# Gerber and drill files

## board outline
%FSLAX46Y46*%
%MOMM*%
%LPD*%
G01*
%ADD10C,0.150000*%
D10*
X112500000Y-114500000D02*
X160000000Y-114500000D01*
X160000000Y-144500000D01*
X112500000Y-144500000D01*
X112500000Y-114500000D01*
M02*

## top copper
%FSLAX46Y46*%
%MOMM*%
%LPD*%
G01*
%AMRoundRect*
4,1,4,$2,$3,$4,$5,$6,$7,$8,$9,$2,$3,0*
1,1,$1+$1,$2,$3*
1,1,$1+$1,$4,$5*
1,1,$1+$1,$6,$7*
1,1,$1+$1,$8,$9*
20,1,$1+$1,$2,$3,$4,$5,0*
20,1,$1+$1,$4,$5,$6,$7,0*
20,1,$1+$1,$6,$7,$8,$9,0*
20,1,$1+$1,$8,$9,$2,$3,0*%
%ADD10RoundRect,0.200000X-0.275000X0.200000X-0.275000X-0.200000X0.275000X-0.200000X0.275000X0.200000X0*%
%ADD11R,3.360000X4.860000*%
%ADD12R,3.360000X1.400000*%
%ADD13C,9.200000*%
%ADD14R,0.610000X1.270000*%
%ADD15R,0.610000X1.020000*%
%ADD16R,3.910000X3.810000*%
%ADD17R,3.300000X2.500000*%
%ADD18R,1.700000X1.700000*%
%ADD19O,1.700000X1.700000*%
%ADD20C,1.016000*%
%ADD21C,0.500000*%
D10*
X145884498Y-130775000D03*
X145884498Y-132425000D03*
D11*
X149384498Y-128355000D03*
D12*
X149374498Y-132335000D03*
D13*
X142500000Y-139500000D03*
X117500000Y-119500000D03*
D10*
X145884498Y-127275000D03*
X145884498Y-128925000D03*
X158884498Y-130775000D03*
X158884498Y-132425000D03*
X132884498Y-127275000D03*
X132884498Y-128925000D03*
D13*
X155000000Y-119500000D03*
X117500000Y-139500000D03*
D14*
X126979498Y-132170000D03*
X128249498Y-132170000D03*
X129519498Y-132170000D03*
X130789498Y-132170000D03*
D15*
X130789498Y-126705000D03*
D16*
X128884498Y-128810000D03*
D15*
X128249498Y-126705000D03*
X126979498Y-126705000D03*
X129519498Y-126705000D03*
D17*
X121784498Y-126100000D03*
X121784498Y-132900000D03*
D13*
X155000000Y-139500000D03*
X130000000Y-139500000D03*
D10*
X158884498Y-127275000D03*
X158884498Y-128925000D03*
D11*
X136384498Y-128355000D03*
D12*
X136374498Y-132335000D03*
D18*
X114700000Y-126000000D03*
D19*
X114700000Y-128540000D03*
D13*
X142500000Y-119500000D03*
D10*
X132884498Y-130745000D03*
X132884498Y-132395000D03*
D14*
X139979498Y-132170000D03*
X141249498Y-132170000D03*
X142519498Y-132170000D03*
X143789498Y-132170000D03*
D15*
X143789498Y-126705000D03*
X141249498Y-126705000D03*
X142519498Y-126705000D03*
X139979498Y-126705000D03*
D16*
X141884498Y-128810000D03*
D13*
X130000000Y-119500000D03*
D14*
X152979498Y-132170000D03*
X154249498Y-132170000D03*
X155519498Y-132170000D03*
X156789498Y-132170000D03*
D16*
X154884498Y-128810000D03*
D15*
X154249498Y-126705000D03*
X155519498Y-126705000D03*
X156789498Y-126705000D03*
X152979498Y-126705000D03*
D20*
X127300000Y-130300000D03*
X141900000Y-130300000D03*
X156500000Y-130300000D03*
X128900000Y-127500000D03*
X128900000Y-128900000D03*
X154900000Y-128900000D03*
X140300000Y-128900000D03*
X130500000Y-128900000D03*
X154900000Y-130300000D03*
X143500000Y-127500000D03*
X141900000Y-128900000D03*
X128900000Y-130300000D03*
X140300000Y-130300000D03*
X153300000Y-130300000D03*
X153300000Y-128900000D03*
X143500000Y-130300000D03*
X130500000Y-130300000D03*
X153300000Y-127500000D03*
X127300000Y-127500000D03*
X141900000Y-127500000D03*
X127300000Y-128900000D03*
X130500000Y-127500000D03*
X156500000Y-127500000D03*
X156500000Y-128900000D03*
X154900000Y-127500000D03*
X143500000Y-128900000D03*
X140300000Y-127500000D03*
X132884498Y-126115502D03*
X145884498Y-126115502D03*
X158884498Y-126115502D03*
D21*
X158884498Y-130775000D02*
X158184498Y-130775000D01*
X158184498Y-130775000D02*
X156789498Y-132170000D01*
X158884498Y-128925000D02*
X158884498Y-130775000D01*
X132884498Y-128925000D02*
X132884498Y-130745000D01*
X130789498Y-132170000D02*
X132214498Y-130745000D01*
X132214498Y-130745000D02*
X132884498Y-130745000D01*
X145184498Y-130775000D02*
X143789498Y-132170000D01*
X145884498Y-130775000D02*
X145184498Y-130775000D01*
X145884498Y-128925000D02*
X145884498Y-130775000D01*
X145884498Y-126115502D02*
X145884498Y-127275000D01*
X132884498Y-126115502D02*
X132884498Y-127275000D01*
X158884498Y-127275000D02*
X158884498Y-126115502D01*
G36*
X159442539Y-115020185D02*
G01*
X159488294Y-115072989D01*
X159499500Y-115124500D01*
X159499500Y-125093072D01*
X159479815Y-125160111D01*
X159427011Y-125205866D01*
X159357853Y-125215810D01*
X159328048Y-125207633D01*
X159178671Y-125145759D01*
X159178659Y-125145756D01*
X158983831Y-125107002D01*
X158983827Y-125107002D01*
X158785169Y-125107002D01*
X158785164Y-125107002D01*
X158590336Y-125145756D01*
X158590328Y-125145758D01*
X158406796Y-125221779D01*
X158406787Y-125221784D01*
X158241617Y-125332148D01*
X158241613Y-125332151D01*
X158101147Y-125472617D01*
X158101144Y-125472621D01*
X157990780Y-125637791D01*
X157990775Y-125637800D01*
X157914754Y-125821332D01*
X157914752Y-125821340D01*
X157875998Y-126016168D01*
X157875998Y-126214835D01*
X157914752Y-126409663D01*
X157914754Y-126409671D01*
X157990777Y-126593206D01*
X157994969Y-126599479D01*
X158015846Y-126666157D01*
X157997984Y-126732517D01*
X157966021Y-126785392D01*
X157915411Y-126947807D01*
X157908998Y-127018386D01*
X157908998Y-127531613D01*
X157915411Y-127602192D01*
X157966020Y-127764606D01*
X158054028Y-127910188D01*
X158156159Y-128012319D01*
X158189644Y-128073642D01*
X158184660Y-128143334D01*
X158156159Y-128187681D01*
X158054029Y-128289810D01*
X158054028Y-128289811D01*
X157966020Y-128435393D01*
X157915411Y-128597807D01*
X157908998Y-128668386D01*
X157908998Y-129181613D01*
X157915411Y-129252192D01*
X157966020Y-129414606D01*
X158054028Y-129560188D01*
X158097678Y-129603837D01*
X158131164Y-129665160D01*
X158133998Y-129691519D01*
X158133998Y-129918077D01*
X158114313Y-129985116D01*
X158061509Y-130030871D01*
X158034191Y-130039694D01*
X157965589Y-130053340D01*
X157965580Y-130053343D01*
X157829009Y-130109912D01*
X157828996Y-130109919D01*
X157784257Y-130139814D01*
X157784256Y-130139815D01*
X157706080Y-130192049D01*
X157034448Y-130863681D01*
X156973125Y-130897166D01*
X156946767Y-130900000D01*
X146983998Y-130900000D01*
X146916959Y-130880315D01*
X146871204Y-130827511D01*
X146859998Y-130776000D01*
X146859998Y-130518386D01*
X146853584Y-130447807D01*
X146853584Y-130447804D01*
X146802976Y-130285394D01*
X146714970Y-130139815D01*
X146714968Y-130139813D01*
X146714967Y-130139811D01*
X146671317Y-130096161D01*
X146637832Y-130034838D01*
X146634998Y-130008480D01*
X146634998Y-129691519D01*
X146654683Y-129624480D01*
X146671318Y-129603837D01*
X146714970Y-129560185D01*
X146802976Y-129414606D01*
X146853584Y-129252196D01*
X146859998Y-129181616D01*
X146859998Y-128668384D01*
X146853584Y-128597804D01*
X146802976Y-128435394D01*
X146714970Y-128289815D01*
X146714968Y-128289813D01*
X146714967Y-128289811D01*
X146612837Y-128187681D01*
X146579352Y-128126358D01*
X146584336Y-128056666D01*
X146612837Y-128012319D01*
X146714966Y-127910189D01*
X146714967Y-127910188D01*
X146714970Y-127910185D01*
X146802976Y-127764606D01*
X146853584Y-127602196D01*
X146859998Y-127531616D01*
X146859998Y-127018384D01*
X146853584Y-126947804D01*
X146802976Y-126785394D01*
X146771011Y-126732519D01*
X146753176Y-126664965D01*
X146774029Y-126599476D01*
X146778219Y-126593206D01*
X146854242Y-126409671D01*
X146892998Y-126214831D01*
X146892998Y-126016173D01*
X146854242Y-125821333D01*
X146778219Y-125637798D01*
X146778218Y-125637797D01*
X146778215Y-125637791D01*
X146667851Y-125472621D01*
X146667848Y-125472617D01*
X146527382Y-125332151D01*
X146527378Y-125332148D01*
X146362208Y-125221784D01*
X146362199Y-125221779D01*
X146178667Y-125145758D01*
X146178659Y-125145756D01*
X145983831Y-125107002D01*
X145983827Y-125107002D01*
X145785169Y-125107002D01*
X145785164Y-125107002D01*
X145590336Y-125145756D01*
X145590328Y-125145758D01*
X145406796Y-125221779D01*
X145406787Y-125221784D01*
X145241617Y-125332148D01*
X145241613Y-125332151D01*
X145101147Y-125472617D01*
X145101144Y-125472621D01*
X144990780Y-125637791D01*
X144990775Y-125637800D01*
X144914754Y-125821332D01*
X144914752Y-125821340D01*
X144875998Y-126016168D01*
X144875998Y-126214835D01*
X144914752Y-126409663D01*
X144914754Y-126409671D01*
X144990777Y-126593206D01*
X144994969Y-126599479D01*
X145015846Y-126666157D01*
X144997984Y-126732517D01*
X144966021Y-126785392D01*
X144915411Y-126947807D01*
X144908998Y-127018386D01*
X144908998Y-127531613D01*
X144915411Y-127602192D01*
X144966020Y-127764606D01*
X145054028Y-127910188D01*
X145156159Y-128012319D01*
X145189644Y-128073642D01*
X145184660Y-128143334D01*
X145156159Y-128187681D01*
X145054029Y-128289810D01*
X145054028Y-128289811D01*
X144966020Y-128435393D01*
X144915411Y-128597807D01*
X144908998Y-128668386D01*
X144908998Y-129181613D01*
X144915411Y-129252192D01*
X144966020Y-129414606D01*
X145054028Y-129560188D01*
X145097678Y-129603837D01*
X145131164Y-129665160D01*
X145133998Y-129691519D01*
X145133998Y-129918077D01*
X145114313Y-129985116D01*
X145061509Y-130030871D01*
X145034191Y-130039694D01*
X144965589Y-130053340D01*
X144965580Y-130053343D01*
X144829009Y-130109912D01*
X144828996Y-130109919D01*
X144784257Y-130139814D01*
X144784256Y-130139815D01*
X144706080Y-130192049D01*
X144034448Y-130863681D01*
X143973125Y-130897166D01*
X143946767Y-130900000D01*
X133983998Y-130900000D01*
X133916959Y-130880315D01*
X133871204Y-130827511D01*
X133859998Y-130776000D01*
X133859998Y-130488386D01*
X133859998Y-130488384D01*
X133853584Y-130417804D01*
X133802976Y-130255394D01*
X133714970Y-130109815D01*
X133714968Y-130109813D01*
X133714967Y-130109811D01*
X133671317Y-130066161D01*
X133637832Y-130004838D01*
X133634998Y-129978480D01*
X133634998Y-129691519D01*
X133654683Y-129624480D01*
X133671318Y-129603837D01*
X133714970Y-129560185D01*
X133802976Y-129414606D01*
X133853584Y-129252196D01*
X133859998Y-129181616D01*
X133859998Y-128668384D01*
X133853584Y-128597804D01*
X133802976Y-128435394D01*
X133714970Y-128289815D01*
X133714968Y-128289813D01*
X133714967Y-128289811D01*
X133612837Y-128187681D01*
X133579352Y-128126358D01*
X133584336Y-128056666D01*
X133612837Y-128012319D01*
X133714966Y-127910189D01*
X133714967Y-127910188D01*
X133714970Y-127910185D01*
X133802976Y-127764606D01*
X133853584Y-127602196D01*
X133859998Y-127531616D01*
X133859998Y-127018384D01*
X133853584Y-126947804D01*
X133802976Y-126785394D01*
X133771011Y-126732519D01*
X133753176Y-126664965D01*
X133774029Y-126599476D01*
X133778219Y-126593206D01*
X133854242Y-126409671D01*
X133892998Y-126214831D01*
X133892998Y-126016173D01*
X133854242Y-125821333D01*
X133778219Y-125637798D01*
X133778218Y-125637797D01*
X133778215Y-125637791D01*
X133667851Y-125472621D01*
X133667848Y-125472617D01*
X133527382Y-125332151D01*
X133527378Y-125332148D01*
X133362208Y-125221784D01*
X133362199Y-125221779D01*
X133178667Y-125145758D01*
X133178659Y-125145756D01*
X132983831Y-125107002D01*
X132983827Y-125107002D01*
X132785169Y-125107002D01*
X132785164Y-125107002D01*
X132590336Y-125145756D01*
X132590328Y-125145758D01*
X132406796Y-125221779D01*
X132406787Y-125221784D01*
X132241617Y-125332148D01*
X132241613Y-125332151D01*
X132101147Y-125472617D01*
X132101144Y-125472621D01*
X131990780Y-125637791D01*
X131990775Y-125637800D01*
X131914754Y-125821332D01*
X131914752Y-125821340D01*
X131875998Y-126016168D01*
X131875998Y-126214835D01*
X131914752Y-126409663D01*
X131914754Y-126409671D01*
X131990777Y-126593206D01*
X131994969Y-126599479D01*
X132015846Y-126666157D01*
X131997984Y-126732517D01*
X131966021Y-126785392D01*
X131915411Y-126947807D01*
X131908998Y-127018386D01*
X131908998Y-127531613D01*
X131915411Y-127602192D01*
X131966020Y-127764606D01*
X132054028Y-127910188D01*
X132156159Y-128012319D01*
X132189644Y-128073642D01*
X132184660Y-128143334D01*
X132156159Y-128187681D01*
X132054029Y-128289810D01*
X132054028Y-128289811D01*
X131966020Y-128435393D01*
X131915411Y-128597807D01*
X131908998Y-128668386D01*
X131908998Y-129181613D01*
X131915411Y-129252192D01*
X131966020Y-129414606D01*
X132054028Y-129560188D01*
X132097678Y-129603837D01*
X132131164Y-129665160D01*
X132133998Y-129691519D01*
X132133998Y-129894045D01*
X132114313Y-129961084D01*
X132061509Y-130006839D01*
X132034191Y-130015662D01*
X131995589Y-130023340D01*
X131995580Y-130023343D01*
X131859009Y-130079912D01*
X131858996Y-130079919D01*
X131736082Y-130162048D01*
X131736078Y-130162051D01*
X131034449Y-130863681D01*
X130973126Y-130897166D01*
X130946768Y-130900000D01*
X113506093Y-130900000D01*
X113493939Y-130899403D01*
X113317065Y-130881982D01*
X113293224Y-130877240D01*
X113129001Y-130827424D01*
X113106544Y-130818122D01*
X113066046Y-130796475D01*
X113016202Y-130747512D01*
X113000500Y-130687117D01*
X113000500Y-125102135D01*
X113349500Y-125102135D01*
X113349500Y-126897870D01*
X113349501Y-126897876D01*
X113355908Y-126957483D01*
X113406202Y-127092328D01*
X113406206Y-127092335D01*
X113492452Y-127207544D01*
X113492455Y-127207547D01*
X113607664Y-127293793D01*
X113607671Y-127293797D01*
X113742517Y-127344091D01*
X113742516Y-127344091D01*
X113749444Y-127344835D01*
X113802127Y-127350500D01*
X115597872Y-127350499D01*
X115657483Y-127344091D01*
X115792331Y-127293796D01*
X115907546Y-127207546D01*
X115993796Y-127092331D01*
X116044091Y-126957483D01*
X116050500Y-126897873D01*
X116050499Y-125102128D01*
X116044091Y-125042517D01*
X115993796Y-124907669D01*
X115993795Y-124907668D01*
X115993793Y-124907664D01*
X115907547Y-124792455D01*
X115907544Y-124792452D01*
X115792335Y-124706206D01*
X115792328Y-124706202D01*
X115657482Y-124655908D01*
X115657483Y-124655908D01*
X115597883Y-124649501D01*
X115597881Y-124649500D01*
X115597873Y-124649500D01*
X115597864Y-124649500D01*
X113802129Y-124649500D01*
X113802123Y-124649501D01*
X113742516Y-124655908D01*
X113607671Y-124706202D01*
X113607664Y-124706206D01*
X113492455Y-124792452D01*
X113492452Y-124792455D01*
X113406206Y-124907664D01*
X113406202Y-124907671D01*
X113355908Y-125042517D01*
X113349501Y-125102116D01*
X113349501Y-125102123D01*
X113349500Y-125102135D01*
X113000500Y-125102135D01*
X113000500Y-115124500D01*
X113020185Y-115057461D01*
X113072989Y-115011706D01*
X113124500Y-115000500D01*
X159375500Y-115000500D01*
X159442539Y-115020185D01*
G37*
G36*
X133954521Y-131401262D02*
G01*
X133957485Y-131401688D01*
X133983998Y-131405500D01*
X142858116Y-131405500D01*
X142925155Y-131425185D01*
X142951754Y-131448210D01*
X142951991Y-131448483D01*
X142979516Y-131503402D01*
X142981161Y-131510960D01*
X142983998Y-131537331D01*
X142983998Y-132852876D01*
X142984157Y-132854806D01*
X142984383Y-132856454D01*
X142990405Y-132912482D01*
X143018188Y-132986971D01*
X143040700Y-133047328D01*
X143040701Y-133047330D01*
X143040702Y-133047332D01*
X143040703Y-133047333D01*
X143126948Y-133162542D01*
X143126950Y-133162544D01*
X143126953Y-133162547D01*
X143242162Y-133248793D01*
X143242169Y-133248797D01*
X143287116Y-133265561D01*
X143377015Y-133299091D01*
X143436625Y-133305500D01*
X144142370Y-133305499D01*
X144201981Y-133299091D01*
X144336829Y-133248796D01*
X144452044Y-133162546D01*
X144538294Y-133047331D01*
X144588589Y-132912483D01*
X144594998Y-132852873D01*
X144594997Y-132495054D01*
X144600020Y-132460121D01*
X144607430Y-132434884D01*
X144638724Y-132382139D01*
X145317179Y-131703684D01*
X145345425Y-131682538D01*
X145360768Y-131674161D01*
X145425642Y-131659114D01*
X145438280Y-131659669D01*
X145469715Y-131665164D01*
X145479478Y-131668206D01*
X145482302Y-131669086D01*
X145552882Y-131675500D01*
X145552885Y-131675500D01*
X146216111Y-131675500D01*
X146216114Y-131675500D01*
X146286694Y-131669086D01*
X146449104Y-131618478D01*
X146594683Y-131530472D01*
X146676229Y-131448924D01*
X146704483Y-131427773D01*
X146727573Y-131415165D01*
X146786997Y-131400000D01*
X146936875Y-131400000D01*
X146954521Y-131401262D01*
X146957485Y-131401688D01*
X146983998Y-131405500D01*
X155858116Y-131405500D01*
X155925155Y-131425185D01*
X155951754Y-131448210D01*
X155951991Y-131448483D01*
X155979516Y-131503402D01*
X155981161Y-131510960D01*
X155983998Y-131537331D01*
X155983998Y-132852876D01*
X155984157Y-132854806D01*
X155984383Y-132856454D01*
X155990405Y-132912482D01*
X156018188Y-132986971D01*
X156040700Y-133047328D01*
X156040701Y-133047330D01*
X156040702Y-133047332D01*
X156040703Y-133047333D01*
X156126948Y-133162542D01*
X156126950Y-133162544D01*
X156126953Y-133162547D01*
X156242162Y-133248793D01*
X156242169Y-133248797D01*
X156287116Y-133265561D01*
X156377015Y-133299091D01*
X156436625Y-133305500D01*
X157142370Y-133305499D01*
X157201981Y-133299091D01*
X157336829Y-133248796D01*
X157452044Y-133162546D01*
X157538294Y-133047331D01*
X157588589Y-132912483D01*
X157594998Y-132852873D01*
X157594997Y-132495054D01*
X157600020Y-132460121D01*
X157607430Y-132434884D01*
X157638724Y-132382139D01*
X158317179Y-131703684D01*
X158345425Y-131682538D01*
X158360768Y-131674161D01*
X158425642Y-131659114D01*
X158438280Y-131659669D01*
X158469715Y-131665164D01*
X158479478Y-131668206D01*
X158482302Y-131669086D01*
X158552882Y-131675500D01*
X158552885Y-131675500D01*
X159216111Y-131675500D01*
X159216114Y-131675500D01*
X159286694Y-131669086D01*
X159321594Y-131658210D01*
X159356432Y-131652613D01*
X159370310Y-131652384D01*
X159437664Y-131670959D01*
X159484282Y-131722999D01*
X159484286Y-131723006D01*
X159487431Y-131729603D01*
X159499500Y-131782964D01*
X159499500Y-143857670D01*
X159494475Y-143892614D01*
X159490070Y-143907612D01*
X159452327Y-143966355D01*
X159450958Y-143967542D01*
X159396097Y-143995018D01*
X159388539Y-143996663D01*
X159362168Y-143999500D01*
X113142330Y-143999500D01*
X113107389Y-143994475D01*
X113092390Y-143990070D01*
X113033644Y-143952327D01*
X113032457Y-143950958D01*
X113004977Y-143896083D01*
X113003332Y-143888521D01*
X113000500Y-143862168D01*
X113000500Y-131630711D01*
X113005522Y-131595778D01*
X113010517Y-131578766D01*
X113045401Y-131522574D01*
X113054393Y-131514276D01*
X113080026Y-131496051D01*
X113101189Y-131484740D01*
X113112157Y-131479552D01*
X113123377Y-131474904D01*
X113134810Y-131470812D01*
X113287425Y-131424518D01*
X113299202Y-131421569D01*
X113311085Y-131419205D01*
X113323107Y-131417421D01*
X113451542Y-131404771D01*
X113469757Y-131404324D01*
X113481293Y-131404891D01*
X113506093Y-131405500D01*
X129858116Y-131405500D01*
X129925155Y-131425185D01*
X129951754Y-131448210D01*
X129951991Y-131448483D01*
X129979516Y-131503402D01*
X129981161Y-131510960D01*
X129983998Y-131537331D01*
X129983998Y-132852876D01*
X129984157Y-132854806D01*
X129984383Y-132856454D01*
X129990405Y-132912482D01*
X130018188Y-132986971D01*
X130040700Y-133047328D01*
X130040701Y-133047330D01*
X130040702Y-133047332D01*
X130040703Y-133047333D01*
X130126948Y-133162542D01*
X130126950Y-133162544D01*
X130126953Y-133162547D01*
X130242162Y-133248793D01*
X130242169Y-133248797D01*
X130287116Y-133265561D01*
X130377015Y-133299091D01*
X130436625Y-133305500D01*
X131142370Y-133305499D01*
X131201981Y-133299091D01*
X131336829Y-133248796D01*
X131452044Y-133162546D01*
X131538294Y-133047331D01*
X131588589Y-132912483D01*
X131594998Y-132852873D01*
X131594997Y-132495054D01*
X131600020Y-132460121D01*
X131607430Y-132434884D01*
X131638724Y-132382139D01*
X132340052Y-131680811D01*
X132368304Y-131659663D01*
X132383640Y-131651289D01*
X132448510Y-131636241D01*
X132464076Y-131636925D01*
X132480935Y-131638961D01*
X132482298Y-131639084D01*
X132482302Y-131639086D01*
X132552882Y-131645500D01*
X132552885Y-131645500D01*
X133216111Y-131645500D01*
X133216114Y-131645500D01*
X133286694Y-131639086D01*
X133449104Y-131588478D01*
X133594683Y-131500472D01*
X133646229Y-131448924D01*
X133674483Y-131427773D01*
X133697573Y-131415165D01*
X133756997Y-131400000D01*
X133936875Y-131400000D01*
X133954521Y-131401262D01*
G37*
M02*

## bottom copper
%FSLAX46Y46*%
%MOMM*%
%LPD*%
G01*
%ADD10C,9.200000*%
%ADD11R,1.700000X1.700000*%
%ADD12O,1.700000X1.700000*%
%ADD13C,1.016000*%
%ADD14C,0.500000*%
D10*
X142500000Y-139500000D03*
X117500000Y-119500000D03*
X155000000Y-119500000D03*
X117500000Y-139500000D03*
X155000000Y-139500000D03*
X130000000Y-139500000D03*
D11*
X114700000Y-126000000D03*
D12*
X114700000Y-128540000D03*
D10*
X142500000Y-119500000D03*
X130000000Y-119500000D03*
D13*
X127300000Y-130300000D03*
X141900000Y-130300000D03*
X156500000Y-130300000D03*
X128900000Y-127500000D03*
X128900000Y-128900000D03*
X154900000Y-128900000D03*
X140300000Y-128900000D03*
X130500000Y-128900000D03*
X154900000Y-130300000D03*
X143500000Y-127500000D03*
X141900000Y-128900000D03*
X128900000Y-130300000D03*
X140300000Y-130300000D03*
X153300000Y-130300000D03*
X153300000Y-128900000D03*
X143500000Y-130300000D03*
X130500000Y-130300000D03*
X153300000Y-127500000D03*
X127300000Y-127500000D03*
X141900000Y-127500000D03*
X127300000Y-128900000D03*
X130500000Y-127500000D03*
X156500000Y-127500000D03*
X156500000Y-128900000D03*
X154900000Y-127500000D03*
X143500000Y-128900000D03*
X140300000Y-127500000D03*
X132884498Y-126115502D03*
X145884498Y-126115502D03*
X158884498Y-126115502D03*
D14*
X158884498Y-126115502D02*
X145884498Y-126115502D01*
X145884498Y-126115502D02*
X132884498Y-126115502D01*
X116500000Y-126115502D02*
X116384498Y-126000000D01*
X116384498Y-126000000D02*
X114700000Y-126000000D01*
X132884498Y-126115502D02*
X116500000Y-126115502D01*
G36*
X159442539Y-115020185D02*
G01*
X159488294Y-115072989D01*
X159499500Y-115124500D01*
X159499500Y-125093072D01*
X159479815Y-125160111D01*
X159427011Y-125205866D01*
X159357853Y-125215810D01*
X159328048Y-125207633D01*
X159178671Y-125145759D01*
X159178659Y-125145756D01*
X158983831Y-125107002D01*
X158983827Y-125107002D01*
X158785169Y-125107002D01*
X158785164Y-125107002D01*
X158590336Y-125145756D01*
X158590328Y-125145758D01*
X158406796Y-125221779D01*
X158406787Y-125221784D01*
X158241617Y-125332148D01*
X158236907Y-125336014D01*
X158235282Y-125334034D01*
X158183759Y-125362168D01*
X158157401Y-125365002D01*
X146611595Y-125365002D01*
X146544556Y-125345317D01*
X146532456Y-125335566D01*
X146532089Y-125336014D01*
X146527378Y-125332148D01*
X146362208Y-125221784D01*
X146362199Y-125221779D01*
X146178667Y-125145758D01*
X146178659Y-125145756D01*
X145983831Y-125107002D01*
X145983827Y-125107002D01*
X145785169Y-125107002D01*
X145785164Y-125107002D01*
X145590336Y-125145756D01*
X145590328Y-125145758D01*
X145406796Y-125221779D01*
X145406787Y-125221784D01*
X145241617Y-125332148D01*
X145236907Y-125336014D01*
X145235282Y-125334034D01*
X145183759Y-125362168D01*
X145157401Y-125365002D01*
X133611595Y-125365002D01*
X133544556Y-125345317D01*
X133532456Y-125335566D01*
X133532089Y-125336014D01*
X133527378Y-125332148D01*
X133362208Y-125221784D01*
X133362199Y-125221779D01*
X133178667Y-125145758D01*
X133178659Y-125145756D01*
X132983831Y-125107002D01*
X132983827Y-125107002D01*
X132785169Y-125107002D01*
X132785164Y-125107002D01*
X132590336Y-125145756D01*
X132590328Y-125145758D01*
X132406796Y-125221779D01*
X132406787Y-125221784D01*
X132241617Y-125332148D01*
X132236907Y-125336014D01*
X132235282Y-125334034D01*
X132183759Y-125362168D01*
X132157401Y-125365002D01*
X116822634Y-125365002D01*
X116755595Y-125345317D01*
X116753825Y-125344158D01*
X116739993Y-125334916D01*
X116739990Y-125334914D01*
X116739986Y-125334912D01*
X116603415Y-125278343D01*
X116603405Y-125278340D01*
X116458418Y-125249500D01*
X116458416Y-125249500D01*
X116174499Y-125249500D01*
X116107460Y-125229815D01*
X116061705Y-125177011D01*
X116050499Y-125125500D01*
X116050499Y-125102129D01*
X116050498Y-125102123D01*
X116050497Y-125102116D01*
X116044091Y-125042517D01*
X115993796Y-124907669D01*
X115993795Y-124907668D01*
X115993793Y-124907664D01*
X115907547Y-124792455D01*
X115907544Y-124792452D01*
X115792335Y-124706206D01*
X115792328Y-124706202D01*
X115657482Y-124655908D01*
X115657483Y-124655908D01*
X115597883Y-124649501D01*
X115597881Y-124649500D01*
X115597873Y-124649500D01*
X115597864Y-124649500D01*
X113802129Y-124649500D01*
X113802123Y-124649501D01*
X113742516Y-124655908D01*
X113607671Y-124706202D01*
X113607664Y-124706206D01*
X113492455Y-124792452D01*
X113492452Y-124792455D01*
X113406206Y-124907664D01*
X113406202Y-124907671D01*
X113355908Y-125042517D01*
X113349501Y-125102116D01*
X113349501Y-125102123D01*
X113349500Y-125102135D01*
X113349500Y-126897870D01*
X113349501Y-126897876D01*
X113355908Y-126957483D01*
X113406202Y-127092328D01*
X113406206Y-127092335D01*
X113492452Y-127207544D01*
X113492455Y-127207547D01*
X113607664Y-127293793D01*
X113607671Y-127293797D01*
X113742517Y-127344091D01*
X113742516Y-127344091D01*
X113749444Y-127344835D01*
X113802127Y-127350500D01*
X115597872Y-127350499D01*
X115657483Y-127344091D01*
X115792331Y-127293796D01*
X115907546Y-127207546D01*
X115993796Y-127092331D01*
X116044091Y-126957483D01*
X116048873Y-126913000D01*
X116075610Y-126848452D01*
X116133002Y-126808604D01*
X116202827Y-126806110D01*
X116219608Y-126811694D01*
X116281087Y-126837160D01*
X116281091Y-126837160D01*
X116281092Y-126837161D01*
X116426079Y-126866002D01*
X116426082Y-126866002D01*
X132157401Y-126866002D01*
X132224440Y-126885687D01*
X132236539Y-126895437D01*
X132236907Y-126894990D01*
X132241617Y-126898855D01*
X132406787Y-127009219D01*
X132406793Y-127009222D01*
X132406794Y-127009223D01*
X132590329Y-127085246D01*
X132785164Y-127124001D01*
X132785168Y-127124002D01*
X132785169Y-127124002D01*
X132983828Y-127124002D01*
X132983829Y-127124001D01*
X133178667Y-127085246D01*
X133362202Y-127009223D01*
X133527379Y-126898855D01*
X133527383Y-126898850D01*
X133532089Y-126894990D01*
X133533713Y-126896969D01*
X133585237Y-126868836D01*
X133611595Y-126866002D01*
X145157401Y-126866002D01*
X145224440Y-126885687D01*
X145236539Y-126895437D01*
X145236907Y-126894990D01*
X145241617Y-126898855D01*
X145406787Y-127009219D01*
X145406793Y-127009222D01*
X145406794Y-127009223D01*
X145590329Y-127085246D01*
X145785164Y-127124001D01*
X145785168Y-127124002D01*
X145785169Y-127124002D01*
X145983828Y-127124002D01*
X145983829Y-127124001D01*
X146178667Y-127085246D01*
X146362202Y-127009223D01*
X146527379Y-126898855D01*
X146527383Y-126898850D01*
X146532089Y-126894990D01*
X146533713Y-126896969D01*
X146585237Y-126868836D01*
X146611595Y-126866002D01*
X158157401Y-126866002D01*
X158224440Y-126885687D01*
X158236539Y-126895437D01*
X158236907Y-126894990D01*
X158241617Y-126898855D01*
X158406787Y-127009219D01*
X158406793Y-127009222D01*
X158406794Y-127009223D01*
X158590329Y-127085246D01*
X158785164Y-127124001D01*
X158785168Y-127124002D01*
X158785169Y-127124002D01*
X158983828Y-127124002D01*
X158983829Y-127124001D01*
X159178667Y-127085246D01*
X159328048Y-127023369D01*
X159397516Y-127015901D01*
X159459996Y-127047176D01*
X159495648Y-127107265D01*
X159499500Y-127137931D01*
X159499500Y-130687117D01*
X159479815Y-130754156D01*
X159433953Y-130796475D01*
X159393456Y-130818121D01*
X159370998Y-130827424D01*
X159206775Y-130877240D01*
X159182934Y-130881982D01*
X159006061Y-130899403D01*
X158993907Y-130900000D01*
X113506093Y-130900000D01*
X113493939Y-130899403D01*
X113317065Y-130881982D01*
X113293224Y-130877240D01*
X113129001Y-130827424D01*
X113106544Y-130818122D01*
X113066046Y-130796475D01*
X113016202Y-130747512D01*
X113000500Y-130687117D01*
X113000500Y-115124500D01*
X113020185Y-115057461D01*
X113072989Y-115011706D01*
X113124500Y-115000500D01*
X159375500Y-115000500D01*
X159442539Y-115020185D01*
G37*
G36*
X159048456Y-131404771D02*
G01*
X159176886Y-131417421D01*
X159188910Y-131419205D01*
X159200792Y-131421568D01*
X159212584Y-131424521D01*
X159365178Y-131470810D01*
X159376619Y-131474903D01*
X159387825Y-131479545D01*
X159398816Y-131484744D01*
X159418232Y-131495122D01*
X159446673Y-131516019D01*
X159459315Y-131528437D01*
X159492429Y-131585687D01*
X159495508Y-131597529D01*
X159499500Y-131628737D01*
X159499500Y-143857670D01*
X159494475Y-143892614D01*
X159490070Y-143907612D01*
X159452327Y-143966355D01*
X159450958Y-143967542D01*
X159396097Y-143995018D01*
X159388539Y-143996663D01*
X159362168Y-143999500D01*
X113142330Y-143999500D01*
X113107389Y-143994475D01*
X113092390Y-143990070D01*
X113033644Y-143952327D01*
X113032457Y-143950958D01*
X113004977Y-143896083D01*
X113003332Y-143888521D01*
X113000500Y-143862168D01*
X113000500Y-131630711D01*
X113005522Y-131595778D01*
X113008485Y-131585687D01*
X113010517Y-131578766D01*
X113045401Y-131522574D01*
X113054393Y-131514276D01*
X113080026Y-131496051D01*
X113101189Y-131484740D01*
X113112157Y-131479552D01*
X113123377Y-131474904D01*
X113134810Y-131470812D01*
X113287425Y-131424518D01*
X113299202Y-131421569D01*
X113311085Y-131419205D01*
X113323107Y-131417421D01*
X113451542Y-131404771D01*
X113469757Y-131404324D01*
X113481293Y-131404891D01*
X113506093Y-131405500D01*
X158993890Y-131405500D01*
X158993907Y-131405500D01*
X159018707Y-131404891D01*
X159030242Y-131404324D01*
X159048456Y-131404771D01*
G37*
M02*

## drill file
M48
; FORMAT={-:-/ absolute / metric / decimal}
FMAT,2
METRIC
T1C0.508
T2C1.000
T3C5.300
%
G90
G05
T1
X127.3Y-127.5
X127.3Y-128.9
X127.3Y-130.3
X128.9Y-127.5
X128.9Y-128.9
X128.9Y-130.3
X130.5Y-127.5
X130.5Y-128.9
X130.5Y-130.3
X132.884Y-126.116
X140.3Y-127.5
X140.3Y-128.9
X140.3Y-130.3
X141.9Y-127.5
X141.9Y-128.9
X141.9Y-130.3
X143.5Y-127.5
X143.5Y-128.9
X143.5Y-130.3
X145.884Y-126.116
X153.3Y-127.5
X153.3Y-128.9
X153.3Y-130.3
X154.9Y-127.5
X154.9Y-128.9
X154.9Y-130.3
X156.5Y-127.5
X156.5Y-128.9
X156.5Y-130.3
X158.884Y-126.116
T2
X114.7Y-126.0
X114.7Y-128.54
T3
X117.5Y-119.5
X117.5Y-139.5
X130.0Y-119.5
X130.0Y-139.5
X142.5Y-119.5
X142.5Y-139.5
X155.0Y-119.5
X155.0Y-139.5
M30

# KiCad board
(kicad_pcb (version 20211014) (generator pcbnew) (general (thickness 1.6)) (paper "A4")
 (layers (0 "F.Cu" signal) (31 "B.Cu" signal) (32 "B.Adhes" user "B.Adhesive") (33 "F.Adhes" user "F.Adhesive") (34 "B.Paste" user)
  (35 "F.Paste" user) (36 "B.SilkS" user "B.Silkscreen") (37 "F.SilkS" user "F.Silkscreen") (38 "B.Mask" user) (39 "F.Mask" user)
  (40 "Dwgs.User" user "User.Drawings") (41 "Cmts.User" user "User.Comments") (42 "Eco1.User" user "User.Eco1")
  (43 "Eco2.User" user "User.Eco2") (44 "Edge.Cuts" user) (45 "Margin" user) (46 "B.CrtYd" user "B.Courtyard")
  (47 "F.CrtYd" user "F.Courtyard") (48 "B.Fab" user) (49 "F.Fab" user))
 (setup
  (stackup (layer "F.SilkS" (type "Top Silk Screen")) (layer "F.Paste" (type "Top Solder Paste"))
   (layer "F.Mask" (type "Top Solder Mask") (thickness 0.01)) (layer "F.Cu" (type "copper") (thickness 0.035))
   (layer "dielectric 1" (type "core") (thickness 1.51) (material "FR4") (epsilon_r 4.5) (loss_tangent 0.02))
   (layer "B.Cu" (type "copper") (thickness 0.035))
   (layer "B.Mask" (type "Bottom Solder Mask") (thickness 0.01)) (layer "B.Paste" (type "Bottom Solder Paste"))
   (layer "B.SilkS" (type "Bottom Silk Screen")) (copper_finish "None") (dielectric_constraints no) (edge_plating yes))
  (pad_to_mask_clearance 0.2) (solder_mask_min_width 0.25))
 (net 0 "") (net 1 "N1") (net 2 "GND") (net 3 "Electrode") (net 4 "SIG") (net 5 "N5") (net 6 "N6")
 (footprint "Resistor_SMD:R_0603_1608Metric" (layer "F.Cu") (at 145.884498 131.6 -90)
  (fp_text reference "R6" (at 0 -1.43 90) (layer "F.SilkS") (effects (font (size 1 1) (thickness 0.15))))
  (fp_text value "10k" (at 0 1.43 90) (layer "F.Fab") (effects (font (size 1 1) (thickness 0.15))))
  (pad "1" smd roundrect (at -0.825 0 270) (size 0.8 0.95) (layers "F.Cu" "F.Paste" "F.Mask") (roundrect_rratio 0.25) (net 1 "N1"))
  (pad "2" smd roundrect (at 0.825 0 270) (size 0.8 0.95) (layers "F.Cu" "F.Paste" "F.Mask") (roundrect_rratio 0.25) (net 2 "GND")))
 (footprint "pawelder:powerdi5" (layer "F.Cu") (at 149.384498 129.625)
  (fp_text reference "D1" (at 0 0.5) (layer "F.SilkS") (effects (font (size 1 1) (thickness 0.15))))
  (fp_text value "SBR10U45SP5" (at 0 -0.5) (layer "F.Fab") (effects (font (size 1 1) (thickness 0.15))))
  (pad "1" smd rect (at 0 -1.27) (size 3.36 4.86) (layers "F.Cu" "F.Paste" "F.Mask") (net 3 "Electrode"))
  (pad "2" smd rect (at -0.01 2.71) (size 3.36 1.4) (layers "F.Cu" "F.Paste" "F.Mask") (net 2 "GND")))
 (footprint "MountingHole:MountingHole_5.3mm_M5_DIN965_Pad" (layer "F.Cu") (at 142.5 139.5)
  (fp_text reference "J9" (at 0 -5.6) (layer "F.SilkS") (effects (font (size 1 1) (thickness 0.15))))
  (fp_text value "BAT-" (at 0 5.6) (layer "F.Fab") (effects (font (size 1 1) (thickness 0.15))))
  (pad "1" thru_hole circle (at 0 0) (size 9.2 9.2) (drill 5.3) (layers *.Cu *.Mask) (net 2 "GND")))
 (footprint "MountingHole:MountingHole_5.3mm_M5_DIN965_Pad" (layer "F.Cu") (at 117.5 119.5)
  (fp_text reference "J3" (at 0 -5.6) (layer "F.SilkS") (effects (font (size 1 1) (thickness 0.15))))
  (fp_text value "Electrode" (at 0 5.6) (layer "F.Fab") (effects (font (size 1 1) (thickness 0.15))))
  (pad "1" thru_hole circle (at 0 0) (size 9.2 9.2) (drill 5.3) (layers *.Cu *.Mask) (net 3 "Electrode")))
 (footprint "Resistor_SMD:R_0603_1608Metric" (layer "F.Cu") (at 145.884498 128.1 -90)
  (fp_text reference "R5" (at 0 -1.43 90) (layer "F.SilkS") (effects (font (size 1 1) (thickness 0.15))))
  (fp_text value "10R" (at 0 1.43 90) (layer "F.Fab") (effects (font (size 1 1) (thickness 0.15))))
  (pad "1" smd roundrect (at -0.825 0 270) (size 0.8 0.95) (layers "F.Cu" "F.Paste" "F.Mask") (roundrect_rratio 0.25) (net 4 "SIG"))
  (pad "2" smd roundrect (at 0.825 0 270) (size 0.8 0.95) (layers "F.Cu" "F.Paste" "F.Mask") (roundrect_rratio 0.25) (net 1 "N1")))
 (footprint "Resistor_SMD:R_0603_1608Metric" (layer "F.Cu") (at 158.884498 131.6 -90)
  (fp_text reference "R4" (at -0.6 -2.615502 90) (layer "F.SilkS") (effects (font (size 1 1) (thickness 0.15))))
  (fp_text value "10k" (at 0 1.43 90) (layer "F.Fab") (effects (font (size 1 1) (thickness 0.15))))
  (pad "1" smd roundrect (at -0.825 0 270) (size 0.8 0.95) (layers "F.Cu" "F.Paste" "F.Mask") (roundrect_rratio 0.25) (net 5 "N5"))
  (pad "2" smd roundrect (at 0.825 0 270) (size 0.8 0.95) (layers "F.Cu" "F.Paste" "F.Mask") (roundrect_rratio 0.25) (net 2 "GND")))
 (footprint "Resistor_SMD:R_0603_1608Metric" (layer "F.Cu") (at 132.884498 128.1 -90)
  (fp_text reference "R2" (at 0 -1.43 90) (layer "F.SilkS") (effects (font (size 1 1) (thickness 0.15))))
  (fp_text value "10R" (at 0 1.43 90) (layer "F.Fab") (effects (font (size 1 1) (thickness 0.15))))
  (pad "1" smd roundrect (at -0.825 0 270) (size 0.8 0.95) (layers "F.Cu" "F.Paste" "F.Mask") (roundrect_rratio 0.25) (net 4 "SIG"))
  (pad "2" smd roundrect (at 0.825 0 270) (size 0.8 0.95) (layers "F.Cu" "F.Paste" "F.Mask") (roundrect_rratio 0.25) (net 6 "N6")))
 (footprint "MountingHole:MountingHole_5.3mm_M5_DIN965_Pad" (layer "F.Cu") (at 155 119.5)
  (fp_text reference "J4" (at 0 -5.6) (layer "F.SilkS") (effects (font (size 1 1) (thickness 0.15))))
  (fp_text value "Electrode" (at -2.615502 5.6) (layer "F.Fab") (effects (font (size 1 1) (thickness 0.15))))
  (pad "1" thru_hole circle (at 0 0) (size 9.2 9.2) (drill 5.3) (layers *.Cu *.Mask) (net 3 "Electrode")))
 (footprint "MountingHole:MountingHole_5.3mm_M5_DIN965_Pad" (layer "F.Cu") (at 117.5 139.5)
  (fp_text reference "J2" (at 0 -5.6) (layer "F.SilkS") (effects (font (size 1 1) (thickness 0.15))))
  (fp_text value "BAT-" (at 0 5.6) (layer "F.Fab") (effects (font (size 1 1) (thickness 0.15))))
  (pad "1" thru_hole circle (at 0 0) (size 9.2 9.2) (drill 5.3) (layers *.Cu *.Mask) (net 2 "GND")))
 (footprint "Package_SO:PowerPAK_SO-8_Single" (layer "F.Cu") (at 128.884498 129.5 90)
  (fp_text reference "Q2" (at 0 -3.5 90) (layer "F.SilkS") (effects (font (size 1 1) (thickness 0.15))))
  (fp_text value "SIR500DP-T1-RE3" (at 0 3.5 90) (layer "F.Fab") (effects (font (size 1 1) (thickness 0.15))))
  (pad "1" smd rect (at -2.67 -1.905 90) (size 1.27 0.61) (layers "F.Cu" "F.Paste" "F.Mask") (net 2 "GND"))
  (pad "2" smd rect (at -2.67 -0.635 90) (size 1.27 0.61) (layers "F.Cu" "F.Paste" "F.Mask") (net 2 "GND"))
  (pad "3" smd rect (at -2.67 0.635 90) (size 1.27 0.61) (layers "F.Cu" "F.Paste" "F.Mask") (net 2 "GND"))
  (pad "4" smd rect (at -2.67 1.905 90) (size 1.27 0.61) (layers "F.Cu" "F.Paste" "F.Mask") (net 6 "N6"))
  (pad "5" smd rect (at 2.795 1.905 90) (size 1.02 0.61) (layers "F.Cu" "F.Paste" "F.Mask") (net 3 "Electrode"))
  (pad "5" smd rect (at 0.69 0 90) (size 3.81 3.91) (layers "F.Cu" "F.Paste" "F.Mask") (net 3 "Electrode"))
  (pad "5" smd rect (at 2.795 -0.635 90) (size 1.02 0.61) (layers "F.Cu" "F.Paste" "F.Mask") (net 3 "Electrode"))
  (pad "5" smd rect (at 2.795 -1.905 90) (size 1.02 0.61) (layers "F.Cu" "F.Paste" "F.Mask") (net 3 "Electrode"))
  (pad "5" smd rect (at 2.795 0.635 90) (size 1.02 0.61) (layers "F.Cu" "F.Paste" "F.Mask") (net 3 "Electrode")))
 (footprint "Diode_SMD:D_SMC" (layer "F.Cu") (at 121.784498 129.5 -90)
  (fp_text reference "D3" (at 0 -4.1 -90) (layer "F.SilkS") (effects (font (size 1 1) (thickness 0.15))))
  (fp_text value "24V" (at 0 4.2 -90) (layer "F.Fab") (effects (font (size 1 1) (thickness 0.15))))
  (pad "1" smd rect (at -3.4 0) (size 3.3 2.5) (layers "F.Cu" "F.Paste" "F.Mask") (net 3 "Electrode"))
  (pad "2" smd rect (at 3.4 0) (size 3.3 2.5) (layers "F.Cu" "F.Paste" "F.Mask") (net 2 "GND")))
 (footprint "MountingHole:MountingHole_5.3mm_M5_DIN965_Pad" (layer "F.Cu") (at 155 139.5)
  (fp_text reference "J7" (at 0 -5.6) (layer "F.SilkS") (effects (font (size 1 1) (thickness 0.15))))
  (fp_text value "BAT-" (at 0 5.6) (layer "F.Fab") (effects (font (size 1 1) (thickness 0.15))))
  (pad "1" thru_hole circle (at 0 0) (size 9.2 9.2) (drill 5.3) (layers *.Cu *.Mask) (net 2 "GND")))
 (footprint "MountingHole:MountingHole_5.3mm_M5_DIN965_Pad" (layer "F.Cu") (at 130 139.5)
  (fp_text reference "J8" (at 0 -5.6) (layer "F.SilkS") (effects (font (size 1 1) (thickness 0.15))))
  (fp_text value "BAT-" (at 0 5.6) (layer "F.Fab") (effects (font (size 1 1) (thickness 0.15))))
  (pad "1" thru_hole circle (at 0 0) (size 9.2 9.2) (drill 5.3) (layers *.Cu *.Mask) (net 2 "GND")))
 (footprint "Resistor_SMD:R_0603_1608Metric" (layer "F.Cu") (at 158.884498 128.1 -90)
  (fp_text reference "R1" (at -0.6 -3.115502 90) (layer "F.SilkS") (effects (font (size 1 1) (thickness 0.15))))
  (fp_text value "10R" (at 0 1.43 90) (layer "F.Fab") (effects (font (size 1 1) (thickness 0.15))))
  (pad "1" smd roundrect (at -0.825 0 270) (size 0.8 0.95) (layers "F.Cu" "F.Paste" "F.Mask") (roundrect_rratio 0.25) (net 4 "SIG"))
  (pad "2" smd roundrect (at 0.825 0 270) (size 0.8 0.95) (layers "F.Cu" "F.Paste" "F.Mask") (roundrect_rratio 0.25) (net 5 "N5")))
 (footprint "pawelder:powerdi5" (layer "F.Cu") (at 136.384498 129.625)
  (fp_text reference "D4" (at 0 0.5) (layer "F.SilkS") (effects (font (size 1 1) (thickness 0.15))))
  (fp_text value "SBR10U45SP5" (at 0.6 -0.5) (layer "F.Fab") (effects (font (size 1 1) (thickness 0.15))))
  (pad "1" smd rect (at 0 -1.27) (size 3.36 4.86) (layers "F.Cu" "F.Paste" "F.Mask") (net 3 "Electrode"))
  (pad "2" smd rect (at -0.01 2.71) (size 3.36 1.4) (layers "F.Cu" "F.Paste" "F.Mask") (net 2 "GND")))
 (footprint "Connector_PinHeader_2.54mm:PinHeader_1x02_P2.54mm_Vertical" (layer "F.Cu") (at 114.7 126)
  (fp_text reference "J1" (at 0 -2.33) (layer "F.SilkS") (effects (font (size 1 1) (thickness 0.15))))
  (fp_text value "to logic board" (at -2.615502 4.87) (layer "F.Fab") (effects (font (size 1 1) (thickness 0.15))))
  (pad "1" thru_hole rect (at 0 0) (size 1.7 1.7) (drill 1) (layers *.Cu *.Mask) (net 4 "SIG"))
  (pad "2" thru_hole oval (at 0 2.54) (size 1.7 1.7) (drill 1) (layers *.Cu *.Mask) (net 3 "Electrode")))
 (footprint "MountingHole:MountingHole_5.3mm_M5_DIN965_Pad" (layer "F.Cu") (at 142.5 119.5)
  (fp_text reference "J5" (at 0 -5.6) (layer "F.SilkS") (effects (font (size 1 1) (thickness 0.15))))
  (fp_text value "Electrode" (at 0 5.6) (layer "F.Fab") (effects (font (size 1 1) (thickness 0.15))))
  (pad "1" thru_hole circle (at 0 0) (size 9.2 9.2) (drill 5.3) (layers *.Cu *.Mask) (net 3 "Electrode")))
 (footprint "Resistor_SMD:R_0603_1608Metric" (layer "F.Cu") (at 132.884498 131.57 -90)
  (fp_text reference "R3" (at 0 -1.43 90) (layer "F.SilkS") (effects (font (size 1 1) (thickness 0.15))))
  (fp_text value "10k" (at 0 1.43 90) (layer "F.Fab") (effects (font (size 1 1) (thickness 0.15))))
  (pad "1" smd roundrect (at -0.825 0 270) (size 0.8 0.95) (layers "F.Cu" "F.Paste" "F.Mask") (roundrect_rratio 0.25) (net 6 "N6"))
  (pad "2" smd roundrect (at 0.825 0 270) (size 0.8 0.95) (layers "F.Cu" "F.Paste" "F.Mask") (roundrect_rratio 0.25) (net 2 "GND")))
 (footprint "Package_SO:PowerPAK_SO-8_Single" (layer "F.Cu") (at 141.884498 129.5 90)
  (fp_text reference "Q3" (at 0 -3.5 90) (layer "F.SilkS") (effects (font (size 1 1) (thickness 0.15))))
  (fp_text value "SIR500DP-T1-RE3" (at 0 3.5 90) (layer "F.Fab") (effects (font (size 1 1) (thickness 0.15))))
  (pad "1" smd rect (at -2.67 -1.905 90) (size 1.27 0.61) (layers "F.Cu" "F.Paste" "F.Mask") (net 2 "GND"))
  (pad "2" smd rect (at -2.67 -0.635 90) (size 1.27 0.61) (layers "F.Cu" "F.Paste" "F.Mask") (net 2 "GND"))
  (pad "3" smd rect (at -2.67 0.635 90) (size 1.27 0.61) (layers "F.Cu" "F.Paste" "F.Mask") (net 2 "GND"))
  (pad "4" smd rect (at -2.67 1.905 90) (size 1.27 0.61) (layers "F.Cu" "F.Paste" "F.Mask") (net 1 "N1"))
  (pad "5" smd rect (at 2.795 1.905 90) (size 1.02 0.61) (layers "F.Cu" "F.Paste" "F.Mask") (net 3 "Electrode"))
  (pad "5" smd rect (at 2.795 -0.635 90) (size 1.02 0.61) (layers "F.Cu" "F.Paste" "F.Mask") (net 3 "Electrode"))
  (pad "5" smd rect (at 2.795 0.635 90) (size 1.02 0.61) (layers "F.Cu" "F.Paste" "F.Mask") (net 3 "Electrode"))
  (pad "5" smd rect (at 2.795 -1.905 90) (size 1.02 0.61) (layers "F.Cu" "F.Paste" "F.Mask") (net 3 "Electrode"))
  (pad "5" smd rect (at 0.69 0 90) (size 3.81 3.91) (layers "F.Cu" "F.Paste" "F.Mask") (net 3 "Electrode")))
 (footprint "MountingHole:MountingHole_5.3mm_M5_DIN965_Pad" (layer "F.Cu") (at 130 119.5)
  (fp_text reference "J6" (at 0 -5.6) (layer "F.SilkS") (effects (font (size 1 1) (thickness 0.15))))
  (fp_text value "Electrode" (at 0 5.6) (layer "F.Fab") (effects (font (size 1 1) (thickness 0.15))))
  (pad "1" thru_hole circle (at 0 0) (size 9.2 9.2) (drill 5.3) (layers *.Cu *.Mask) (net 3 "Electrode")))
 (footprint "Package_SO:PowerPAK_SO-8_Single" (layer "F.Cu") (at 154.884498 129.5 90)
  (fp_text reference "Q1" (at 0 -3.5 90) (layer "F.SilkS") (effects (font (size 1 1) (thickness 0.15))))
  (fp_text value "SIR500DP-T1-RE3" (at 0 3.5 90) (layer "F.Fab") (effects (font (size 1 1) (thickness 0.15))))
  (pad "1" smd rect (at -2.67 -1.905 90) (size 1.27 0.61) (layers "F.Cu" "F.Paste" "F.Mask") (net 2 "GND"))
  (pad "2" smd rect (at -2.67 -0.635 90) (size 1.27 0.61) (layers "F.Cu" "F.Paste" "F.Mask") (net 2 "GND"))
  (pad "3" smd rect (at -2.67 0.635 90) (size 1.27 0.61) (layers "F.Cu" "F.Paste" "F.Mask") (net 2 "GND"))
  (pad "4" smd rect (at -2.67 1.905 90) (size 1.27 0.61) (layers "F.Cu" "F.Paste" "F.Mask") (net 5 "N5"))
  (pad "5" smd rect (at 0.69 0 90) (size 3.81 3.91) (layers "F.Cu" "F.Paste" "F.Mask") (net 3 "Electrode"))
  (pad "5" smd rect (at 2.795 -0.635 90) (size 1.02 0.61) (layers "F.Cu" "F.Paste" "F.Mask") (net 3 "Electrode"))
  (pad "5" smd rect (at 2.795 0.635 90) (size 1.02 0.61) (layers "F.Cu" "F.Paste" "F.Mask") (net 3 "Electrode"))
  (pad "5" smd rect (at 2.795 1.905 90) (size 1.02 0.61) (layers "F.Cu" "F.Paste" "F.Mask") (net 3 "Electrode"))
  (pad "5" smd rect (at 2.795 -1.905 90) (size 1.02 0.61) (layers "F.Cu" "F.Paste" "F.Mask") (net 3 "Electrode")))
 (gr_rect (start 112.5 114.5) (end 160 144.5) (layer "Edge.Cuts") (width 0.15) (fill none))
 (via (at 127.3 130.3) (size 1.016) (drill 0.508) (layers "F.Cu" "B.Cu") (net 3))
 (via (at 141.9 130.3) (size 1.016) (drill 0.508) (layers "F.Cu" "B.Cu") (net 3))
 (via (at 156.5 130.3) (size 1.016) (drill 0.508) (layers "F.Cu" "B.Cu") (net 3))
 (via (at 128.9 127.5) (size 1.016) (drill 0.508) (layers "F.Cu" "B.Cu") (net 3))
 (via (at 128.9 128.9) (size 1.016) (drill 0.508) (layers "F.Cu" "B.Cu") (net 3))
 (via (at 154.9 128.9) (size 1.016) (drill 0.508) (layers "F.Cu" "B.Cu") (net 3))
 (via (at 140.3 128.9) (size 1.016) (drill 0.508) (layers "F.Cu" "B.Cu") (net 3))
 (via (at 130.5 128.9) (size 1.016) (drill 0.508) (layers "F.Cu" "B.Cu") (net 3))
 (via (at 154.9 130.3) (size 1.016) (drill 0.508) (layers "F.Cu" "B.Cu") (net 3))
 (via (at 143.5 127.5) (size 1.016) (drill 0.508) (layers "F.Cu" "B.Cu") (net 3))
 (via (at 141.9 128.9) (size 1.016) (drill 0.508) (layers "F.Cu" "B.Cu") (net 3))
 (via (at 128.9 130.3) (size 1.016) (drill 0.508) (layers "F.Cu" "B.Cu") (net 3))
 (via (at 140.3 130.3) (size 1.016) (drill 0.508) (layers "F.Cu" "B.Cu") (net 3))
 (via (at 153.3 130.3) (size 1.016) (drill 0.508) (layers "F.Cu" "B.Cu") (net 3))
 (via (at 153.3 128.9) (size 1.016) (drill 0.508) (layers "F.Cu" "B.Cu") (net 3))
 (via (at 143.5 130.3) (size 1.016) (drill 0.508) (layers "F.Cu" "B.Cu") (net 3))
 (via (at 130.5 130.3) (size 1.016) (drill 0.508) (layers "F.Cu" "B.Cu") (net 3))
 (via (at 153.3 127.5) (size 1.016) (drill 0.508) (layers "F.Cu" "B.Cu") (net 3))
 (via (at 127.3 127.5) (size 1.016) (drill 0.508) (layers "F.Cu" "B.Cu") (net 3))
 (via (at 141.9 127.5) (size 1.016) (drill 0.508) (layers "F.Cu" "B.Cu") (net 3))
 (via (at 127.3 128.9) (size 1.016) (drill 0.508) (layers "F.Cu" "B.Cu") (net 3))
 (via (at 130.5 127.5) (size 1.016) (drill 0.508) (layers "F.Cu" "B.Cu") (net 3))
 (via (at 156.5 127.5) (size 1.016) (drill 0.508) (layers "F.Cu" "B.Cu") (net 3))
 (via (at 156.5 128.9) (size 1.016) (drill 0.508) (layers "F.Cu" "B.Cu") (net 3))
 (via (at 154.9 127.5) (size 1.016) (drill 0.508) (layers "F.Cu" "B.Cu") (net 3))
 (via (at 143.5 128.9) (size 1.016) (drill 0.508) (layers "F.Cu" "B.Cu") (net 3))
 (via (at 140.3 127.5) (size 1.016) (drill 0.508) (layers "F.Cu" "B.Cu") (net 3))
 (segment (start 158.884498 130.775) (end 158.184498 130.775) (width 0.5) (layer "F.Cu") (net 5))
 (segment (start 158.184498 130.775) (end 156.789498 132.17) (width 0.5) (layer "F.Cu") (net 5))
 (segment (start 158.884498 128.925) (end 158.884498 130.775) (width 0.5) (layer "F.Cu") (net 5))
 (segment (start 132.884498 128.925) (end 132.884498 130.745) (width 0.5) (layer "F.Cu") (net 6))
 (segment (start 130.789498 132.17) (end 132.214498 130.745) (width 0.5) (layer "F.Cu") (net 6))
 (segment (start 132.214498 130.745) (end 132.884498 130.745) (width 0.5) (layer "F.Cu") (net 6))
 (segment (start 145.184498 130.775) (end 143.789498 132.17) (width 0.5) (layer "F.Cu") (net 1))
 (segment (start 145.884498 130.775) (end 145.184498 130.775) (width 0.5) (layer "F.Cu") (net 1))
 (segment (start 145.884498 128.925) (end 145.884498 130.775) (width 0.5) (layer "F.Cu") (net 1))
 (segment (start 145.884498 126.115502) (end 145.884498 127.275) (width 0.5) (layer "F.Cu") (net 4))
 (segment (start 132.884498 126.115502) (end 132.884498 127.275) (width 0.5) (layer "F.Cu") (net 4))
 (segment (start 158.884498 127.275) (end 158.884498 126.115502) (width 0.5) (layer "F.Cu") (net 4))
 (via (at 132.884498 126.115502) (size 1.016) (drill 0.508) (layers "F.Cu" "B.Cu") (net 4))
 (via (at 145.884498 126.115502) (size 1.016) (drill 0.508) (layers "F.Cu" "B.Cu") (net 4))
 (via (at 158.884498 126.115502) (size 1.016) (drill 0.508) (layers "F.Cu" "B.Cu") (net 4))
 (segment (start 158.884498 126.115502) (end 145.884498 126.115502) (width 0.5) (layer "B.Cu") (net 4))
 (segment (start 145.884498 126.115502) (end 132.884498 126.115502) (width 0.5) (layer "B.Cu") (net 4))
 (segment (start 116.5 126.115502) (end 116.384498 126) (width 0.5) (layer "B.Cu") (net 4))
 (segment (start 116.384498 126) (end 114.7 126) (width 0.5) (layer "B.Cu") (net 4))
 (segment (start 132.884498 126.115502) (end 116.5 126.115502) (width 0.5) (layer "B.Cu") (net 4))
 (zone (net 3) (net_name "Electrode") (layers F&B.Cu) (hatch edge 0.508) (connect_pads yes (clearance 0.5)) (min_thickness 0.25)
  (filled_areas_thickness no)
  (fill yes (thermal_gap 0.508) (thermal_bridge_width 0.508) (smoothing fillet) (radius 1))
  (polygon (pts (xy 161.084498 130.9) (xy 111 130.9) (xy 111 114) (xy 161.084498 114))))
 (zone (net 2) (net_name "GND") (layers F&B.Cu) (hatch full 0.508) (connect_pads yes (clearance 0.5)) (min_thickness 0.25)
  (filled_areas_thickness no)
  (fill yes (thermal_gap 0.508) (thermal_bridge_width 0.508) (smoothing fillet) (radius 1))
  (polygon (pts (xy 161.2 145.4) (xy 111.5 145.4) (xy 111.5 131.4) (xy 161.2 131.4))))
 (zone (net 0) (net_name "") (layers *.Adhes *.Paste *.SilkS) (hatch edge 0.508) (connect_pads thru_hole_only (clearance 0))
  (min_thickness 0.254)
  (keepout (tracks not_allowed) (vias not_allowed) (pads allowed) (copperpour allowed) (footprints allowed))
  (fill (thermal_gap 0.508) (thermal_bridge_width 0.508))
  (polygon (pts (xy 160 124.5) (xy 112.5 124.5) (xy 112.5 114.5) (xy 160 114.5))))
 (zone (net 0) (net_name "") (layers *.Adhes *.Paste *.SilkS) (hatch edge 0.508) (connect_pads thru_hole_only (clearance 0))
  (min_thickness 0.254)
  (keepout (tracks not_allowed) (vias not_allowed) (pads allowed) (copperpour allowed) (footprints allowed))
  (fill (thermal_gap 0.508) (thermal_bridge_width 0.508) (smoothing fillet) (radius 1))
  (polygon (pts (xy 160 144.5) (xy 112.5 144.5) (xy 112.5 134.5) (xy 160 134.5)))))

